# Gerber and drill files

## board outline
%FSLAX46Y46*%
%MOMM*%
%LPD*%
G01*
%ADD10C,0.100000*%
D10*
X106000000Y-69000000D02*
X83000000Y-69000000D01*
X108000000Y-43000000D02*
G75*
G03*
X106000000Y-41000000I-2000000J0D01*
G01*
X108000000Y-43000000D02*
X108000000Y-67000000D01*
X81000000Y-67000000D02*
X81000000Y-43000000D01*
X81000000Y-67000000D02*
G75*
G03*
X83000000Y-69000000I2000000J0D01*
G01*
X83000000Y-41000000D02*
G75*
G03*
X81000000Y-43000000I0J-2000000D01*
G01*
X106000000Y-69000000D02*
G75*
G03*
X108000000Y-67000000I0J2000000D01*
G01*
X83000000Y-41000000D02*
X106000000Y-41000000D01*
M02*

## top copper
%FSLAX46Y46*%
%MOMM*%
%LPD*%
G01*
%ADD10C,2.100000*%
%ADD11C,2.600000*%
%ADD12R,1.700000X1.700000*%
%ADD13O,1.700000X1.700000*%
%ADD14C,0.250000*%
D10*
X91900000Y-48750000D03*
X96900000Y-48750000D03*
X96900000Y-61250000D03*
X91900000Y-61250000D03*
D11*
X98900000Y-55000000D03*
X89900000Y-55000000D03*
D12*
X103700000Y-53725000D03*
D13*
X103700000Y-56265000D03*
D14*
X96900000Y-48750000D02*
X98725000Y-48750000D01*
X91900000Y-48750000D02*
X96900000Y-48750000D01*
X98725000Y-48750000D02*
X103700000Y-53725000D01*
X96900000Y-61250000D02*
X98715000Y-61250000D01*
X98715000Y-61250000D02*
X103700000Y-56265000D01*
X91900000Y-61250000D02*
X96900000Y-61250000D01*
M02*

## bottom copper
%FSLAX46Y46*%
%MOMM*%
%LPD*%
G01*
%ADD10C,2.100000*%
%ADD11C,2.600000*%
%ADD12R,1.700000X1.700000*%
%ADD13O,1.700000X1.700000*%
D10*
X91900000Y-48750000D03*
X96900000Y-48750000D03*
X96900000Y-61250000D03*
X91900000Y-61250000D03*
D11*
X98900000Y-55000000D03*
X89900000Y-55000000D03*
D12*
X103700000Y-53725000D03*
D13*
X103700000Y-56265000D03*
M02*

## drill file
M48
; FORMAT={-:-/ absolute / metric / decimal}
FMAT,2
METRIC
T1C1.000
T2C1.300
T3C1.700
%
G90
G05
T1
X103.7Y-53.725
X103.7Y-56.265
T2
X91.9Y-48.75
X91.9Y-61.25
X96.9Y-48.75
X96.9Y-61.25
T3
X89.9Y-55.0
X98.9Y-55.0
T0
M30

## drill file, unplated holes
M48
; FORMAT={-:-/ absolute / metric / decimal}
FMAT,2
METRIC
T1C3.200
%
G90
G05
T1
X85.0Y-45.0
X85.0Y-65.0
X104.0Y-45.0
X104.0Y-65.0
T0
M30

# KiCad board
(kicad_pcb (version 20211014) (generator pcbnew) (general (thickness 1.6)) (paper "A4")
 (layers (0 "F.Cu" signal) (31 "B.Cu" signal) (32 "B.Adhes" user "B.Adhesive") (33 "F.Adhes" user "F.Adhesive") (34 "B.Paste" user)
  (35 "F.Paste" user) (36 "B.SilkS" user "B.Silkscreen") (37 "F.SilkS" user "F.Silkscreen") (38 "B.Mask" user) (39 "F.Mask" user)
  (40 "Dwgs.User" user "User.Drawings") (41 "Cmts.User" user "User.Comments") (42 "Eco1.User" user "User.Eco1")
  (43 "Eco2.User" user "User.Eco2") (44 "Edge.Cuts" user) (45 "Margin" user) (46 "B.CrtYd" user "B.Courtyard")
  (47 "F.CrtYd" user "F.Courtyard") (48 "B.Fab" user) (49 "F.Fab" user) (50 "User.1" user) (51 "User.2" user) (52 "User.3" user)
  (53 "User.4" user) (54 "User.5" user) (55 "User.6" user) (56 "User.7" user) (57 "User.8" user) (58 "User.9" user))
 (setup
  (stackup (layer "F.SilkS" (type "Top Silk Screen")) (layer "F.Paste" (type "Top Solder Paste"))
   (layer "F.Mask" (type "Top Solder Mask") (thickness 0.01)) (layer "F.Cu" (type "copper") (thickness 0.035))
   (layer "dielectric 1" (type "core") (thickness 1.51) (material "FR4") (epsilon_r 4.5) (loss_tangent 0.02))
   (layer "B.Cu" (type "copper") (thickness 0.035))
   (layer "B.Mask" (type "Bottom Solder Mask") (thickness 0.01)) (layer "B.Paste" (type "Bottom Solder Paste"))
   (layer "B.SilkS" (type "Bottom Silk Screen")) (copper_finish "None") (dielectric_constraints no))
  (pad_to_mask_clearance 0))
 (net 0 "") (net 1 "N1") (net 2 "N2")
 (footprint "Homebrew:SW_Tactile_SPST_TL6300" (layer "F.Cu") (at 91.9 48.75) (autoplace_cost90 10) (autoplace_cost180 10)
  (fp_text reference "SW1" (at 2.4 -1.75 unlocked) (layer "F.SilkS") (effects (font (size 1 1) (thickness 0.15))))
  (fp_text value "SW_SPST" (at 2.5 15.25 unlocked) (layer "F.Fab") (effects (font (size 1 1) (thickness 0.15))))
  (pad "1" thru_hole circle (at 0 0) (size 2.1 2.1) (drill 1.3) (layers *.Cu *.Mask) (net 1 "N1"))
  (pad "1" thru_hole circle (at 5 0) (size 2.1 2.1) (drill 1.3) (layers *.Cu *.Mask) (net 1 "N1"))
  (pad "2" thru_hole circle (at 5 12.5) (size 2.1 2.1) (drill 1.3) (layers *.Cu *.Mask) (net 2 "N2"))
  (pad "2" thru_hole circle (at 0 12.5) (size 2.1 2.1) (drill 1.3) (layers *.Cu *.Mask) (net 2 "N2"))
  (pad "~" thru_hole circle (at 7 6.25) (size 2.6 2.6) (drill 1.7) (layers *.Cu *.Mask))
  (pad "~" thru_hole circle (at -2 6.25) (size 2.6 2.6) (drill 1.7) (layers *.Cu *.Mask)))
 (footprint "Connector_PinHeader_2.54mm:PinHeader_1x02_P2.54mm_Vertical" (layer "F.Cu") (at 103.7 53.725)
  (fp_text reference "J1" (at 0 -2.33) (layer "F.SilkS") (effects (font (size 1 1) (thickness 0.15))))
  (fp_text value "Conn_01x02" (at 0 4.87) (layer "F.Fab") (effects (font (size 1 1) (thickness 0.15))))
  (pad "1" thru_hole rect (at 0 0) (size 1.7 1.7) (drill 1) (layers *.Cu *.Mask) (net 1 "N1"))
  (pad "2" thru_hole oval (at 0 2.54) (size 1.7 1.7) (drill 1) (layers *.Cu *.Mask) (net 2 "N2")))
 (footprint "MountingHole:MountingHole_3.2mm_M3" (layer "F.Cu") (at 104 45)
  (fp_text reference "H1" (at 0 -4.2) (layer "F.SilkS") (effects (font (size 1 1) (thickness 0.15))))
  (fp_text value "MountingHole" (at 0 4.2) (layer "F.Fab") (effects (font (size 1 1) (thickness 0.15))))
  (pad "" np_thru_hole circle (at 0 0) (size 3.2 3.2) (drill 3.2) (layers *.Cu *.Mask)))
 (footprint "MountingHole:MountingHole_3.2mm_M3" (layer "F.Cu") (at 85 45)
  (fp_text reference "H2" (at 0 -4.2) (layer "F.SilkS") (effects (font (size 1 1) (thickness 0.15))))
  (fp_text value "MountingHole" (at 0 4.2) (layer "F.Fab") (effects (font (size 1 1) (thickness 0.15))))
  (pad "" np_thru_hole circle (at 0 0) (size 3.2 3.2) (drill 3.2) (layers *.Cu *.Mask)))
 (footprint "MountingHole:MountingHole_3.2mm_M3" (layer "F.Cu") (at 104 65)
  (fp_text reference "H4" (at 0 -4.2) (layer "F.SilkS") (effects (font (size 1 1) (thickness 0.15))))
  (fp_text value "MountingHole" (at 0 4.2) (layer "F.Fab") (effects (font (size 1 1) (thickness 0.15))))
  (pad "" np_thru_hole circle (at 0 0) (size 3.2 3.2) (drill 3.2) (layers *.Cu *.Mask)))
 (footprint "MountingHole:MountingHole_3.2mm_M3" (layer "F.Cu") (at 85 65)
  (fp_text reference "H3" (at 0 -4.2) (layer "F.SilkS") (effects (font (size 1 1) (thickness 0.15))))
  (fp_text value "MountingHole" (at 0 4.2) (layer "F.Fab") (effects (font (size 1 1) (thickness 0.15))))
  (pad "" np_thru_hole circle (at 0 0) (size 3.2 3.2) (drill 3.2) (layers *.Cu *.Mask)))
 (gr_line (start 106 69) (end 83 69) (layer "Edge.Cuts") (width 0.1))
 (gr_arc (start 106 41) (mid 107.414214 41.585786) (end 108 43) (layer "Edge.Cuts") (width 0.1))
 (gr_line (start 108 43) (end 108 67) (layer "Edge.Cuts") (width 0.1))
 (gr_line (start 81 67) (end 81 43) (layer "Edge.Cuts") (width 0.1))
 (gr_arc (start 83 69) (mid 81.585786 68.414214) (end 81 67) (layer "Edge.Cuts") (width 0.1))
 (gr_arc (start 81 43) (mid 81.585786 41.585786) (end 83 41) (layer "Edge.Cuts") (width 0.1))
 (gr_arc (start 108 67) (mid 107.414214 68.414214) (end 106 69) (layer "Edge.Cuts") (width 0.1))
 (gr_line (start 83 41) (end 106 41) (layer "Edge.Cuts") (width 0.1))
 (segment (start 96.9 48.75) (end 98.725 48.75) (width 0.25) (layer "F.Cu") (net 1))
 (segment (start 91.9 48.75) (end 96.9 48.75) (width 0.25) (layer "F.Cu") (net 1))
 (segment (start 98.725 48.75) (end 103.7 53.725) (width 0.25) (layer "F.Cu") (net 1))
 (segment (start 96.9 61.25) (end 98.715 61.25) (width 0.25) (layer "F.Cu") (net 2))
 (segment (start 98.715 61.25) (end 103.7 56.265) (width 0.25) (layer "F.Cu") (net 2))
 (segment (start 91.9 61.25) (end 96.9 61.25) (width 0.25) (layer "F.Cu") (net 2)))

